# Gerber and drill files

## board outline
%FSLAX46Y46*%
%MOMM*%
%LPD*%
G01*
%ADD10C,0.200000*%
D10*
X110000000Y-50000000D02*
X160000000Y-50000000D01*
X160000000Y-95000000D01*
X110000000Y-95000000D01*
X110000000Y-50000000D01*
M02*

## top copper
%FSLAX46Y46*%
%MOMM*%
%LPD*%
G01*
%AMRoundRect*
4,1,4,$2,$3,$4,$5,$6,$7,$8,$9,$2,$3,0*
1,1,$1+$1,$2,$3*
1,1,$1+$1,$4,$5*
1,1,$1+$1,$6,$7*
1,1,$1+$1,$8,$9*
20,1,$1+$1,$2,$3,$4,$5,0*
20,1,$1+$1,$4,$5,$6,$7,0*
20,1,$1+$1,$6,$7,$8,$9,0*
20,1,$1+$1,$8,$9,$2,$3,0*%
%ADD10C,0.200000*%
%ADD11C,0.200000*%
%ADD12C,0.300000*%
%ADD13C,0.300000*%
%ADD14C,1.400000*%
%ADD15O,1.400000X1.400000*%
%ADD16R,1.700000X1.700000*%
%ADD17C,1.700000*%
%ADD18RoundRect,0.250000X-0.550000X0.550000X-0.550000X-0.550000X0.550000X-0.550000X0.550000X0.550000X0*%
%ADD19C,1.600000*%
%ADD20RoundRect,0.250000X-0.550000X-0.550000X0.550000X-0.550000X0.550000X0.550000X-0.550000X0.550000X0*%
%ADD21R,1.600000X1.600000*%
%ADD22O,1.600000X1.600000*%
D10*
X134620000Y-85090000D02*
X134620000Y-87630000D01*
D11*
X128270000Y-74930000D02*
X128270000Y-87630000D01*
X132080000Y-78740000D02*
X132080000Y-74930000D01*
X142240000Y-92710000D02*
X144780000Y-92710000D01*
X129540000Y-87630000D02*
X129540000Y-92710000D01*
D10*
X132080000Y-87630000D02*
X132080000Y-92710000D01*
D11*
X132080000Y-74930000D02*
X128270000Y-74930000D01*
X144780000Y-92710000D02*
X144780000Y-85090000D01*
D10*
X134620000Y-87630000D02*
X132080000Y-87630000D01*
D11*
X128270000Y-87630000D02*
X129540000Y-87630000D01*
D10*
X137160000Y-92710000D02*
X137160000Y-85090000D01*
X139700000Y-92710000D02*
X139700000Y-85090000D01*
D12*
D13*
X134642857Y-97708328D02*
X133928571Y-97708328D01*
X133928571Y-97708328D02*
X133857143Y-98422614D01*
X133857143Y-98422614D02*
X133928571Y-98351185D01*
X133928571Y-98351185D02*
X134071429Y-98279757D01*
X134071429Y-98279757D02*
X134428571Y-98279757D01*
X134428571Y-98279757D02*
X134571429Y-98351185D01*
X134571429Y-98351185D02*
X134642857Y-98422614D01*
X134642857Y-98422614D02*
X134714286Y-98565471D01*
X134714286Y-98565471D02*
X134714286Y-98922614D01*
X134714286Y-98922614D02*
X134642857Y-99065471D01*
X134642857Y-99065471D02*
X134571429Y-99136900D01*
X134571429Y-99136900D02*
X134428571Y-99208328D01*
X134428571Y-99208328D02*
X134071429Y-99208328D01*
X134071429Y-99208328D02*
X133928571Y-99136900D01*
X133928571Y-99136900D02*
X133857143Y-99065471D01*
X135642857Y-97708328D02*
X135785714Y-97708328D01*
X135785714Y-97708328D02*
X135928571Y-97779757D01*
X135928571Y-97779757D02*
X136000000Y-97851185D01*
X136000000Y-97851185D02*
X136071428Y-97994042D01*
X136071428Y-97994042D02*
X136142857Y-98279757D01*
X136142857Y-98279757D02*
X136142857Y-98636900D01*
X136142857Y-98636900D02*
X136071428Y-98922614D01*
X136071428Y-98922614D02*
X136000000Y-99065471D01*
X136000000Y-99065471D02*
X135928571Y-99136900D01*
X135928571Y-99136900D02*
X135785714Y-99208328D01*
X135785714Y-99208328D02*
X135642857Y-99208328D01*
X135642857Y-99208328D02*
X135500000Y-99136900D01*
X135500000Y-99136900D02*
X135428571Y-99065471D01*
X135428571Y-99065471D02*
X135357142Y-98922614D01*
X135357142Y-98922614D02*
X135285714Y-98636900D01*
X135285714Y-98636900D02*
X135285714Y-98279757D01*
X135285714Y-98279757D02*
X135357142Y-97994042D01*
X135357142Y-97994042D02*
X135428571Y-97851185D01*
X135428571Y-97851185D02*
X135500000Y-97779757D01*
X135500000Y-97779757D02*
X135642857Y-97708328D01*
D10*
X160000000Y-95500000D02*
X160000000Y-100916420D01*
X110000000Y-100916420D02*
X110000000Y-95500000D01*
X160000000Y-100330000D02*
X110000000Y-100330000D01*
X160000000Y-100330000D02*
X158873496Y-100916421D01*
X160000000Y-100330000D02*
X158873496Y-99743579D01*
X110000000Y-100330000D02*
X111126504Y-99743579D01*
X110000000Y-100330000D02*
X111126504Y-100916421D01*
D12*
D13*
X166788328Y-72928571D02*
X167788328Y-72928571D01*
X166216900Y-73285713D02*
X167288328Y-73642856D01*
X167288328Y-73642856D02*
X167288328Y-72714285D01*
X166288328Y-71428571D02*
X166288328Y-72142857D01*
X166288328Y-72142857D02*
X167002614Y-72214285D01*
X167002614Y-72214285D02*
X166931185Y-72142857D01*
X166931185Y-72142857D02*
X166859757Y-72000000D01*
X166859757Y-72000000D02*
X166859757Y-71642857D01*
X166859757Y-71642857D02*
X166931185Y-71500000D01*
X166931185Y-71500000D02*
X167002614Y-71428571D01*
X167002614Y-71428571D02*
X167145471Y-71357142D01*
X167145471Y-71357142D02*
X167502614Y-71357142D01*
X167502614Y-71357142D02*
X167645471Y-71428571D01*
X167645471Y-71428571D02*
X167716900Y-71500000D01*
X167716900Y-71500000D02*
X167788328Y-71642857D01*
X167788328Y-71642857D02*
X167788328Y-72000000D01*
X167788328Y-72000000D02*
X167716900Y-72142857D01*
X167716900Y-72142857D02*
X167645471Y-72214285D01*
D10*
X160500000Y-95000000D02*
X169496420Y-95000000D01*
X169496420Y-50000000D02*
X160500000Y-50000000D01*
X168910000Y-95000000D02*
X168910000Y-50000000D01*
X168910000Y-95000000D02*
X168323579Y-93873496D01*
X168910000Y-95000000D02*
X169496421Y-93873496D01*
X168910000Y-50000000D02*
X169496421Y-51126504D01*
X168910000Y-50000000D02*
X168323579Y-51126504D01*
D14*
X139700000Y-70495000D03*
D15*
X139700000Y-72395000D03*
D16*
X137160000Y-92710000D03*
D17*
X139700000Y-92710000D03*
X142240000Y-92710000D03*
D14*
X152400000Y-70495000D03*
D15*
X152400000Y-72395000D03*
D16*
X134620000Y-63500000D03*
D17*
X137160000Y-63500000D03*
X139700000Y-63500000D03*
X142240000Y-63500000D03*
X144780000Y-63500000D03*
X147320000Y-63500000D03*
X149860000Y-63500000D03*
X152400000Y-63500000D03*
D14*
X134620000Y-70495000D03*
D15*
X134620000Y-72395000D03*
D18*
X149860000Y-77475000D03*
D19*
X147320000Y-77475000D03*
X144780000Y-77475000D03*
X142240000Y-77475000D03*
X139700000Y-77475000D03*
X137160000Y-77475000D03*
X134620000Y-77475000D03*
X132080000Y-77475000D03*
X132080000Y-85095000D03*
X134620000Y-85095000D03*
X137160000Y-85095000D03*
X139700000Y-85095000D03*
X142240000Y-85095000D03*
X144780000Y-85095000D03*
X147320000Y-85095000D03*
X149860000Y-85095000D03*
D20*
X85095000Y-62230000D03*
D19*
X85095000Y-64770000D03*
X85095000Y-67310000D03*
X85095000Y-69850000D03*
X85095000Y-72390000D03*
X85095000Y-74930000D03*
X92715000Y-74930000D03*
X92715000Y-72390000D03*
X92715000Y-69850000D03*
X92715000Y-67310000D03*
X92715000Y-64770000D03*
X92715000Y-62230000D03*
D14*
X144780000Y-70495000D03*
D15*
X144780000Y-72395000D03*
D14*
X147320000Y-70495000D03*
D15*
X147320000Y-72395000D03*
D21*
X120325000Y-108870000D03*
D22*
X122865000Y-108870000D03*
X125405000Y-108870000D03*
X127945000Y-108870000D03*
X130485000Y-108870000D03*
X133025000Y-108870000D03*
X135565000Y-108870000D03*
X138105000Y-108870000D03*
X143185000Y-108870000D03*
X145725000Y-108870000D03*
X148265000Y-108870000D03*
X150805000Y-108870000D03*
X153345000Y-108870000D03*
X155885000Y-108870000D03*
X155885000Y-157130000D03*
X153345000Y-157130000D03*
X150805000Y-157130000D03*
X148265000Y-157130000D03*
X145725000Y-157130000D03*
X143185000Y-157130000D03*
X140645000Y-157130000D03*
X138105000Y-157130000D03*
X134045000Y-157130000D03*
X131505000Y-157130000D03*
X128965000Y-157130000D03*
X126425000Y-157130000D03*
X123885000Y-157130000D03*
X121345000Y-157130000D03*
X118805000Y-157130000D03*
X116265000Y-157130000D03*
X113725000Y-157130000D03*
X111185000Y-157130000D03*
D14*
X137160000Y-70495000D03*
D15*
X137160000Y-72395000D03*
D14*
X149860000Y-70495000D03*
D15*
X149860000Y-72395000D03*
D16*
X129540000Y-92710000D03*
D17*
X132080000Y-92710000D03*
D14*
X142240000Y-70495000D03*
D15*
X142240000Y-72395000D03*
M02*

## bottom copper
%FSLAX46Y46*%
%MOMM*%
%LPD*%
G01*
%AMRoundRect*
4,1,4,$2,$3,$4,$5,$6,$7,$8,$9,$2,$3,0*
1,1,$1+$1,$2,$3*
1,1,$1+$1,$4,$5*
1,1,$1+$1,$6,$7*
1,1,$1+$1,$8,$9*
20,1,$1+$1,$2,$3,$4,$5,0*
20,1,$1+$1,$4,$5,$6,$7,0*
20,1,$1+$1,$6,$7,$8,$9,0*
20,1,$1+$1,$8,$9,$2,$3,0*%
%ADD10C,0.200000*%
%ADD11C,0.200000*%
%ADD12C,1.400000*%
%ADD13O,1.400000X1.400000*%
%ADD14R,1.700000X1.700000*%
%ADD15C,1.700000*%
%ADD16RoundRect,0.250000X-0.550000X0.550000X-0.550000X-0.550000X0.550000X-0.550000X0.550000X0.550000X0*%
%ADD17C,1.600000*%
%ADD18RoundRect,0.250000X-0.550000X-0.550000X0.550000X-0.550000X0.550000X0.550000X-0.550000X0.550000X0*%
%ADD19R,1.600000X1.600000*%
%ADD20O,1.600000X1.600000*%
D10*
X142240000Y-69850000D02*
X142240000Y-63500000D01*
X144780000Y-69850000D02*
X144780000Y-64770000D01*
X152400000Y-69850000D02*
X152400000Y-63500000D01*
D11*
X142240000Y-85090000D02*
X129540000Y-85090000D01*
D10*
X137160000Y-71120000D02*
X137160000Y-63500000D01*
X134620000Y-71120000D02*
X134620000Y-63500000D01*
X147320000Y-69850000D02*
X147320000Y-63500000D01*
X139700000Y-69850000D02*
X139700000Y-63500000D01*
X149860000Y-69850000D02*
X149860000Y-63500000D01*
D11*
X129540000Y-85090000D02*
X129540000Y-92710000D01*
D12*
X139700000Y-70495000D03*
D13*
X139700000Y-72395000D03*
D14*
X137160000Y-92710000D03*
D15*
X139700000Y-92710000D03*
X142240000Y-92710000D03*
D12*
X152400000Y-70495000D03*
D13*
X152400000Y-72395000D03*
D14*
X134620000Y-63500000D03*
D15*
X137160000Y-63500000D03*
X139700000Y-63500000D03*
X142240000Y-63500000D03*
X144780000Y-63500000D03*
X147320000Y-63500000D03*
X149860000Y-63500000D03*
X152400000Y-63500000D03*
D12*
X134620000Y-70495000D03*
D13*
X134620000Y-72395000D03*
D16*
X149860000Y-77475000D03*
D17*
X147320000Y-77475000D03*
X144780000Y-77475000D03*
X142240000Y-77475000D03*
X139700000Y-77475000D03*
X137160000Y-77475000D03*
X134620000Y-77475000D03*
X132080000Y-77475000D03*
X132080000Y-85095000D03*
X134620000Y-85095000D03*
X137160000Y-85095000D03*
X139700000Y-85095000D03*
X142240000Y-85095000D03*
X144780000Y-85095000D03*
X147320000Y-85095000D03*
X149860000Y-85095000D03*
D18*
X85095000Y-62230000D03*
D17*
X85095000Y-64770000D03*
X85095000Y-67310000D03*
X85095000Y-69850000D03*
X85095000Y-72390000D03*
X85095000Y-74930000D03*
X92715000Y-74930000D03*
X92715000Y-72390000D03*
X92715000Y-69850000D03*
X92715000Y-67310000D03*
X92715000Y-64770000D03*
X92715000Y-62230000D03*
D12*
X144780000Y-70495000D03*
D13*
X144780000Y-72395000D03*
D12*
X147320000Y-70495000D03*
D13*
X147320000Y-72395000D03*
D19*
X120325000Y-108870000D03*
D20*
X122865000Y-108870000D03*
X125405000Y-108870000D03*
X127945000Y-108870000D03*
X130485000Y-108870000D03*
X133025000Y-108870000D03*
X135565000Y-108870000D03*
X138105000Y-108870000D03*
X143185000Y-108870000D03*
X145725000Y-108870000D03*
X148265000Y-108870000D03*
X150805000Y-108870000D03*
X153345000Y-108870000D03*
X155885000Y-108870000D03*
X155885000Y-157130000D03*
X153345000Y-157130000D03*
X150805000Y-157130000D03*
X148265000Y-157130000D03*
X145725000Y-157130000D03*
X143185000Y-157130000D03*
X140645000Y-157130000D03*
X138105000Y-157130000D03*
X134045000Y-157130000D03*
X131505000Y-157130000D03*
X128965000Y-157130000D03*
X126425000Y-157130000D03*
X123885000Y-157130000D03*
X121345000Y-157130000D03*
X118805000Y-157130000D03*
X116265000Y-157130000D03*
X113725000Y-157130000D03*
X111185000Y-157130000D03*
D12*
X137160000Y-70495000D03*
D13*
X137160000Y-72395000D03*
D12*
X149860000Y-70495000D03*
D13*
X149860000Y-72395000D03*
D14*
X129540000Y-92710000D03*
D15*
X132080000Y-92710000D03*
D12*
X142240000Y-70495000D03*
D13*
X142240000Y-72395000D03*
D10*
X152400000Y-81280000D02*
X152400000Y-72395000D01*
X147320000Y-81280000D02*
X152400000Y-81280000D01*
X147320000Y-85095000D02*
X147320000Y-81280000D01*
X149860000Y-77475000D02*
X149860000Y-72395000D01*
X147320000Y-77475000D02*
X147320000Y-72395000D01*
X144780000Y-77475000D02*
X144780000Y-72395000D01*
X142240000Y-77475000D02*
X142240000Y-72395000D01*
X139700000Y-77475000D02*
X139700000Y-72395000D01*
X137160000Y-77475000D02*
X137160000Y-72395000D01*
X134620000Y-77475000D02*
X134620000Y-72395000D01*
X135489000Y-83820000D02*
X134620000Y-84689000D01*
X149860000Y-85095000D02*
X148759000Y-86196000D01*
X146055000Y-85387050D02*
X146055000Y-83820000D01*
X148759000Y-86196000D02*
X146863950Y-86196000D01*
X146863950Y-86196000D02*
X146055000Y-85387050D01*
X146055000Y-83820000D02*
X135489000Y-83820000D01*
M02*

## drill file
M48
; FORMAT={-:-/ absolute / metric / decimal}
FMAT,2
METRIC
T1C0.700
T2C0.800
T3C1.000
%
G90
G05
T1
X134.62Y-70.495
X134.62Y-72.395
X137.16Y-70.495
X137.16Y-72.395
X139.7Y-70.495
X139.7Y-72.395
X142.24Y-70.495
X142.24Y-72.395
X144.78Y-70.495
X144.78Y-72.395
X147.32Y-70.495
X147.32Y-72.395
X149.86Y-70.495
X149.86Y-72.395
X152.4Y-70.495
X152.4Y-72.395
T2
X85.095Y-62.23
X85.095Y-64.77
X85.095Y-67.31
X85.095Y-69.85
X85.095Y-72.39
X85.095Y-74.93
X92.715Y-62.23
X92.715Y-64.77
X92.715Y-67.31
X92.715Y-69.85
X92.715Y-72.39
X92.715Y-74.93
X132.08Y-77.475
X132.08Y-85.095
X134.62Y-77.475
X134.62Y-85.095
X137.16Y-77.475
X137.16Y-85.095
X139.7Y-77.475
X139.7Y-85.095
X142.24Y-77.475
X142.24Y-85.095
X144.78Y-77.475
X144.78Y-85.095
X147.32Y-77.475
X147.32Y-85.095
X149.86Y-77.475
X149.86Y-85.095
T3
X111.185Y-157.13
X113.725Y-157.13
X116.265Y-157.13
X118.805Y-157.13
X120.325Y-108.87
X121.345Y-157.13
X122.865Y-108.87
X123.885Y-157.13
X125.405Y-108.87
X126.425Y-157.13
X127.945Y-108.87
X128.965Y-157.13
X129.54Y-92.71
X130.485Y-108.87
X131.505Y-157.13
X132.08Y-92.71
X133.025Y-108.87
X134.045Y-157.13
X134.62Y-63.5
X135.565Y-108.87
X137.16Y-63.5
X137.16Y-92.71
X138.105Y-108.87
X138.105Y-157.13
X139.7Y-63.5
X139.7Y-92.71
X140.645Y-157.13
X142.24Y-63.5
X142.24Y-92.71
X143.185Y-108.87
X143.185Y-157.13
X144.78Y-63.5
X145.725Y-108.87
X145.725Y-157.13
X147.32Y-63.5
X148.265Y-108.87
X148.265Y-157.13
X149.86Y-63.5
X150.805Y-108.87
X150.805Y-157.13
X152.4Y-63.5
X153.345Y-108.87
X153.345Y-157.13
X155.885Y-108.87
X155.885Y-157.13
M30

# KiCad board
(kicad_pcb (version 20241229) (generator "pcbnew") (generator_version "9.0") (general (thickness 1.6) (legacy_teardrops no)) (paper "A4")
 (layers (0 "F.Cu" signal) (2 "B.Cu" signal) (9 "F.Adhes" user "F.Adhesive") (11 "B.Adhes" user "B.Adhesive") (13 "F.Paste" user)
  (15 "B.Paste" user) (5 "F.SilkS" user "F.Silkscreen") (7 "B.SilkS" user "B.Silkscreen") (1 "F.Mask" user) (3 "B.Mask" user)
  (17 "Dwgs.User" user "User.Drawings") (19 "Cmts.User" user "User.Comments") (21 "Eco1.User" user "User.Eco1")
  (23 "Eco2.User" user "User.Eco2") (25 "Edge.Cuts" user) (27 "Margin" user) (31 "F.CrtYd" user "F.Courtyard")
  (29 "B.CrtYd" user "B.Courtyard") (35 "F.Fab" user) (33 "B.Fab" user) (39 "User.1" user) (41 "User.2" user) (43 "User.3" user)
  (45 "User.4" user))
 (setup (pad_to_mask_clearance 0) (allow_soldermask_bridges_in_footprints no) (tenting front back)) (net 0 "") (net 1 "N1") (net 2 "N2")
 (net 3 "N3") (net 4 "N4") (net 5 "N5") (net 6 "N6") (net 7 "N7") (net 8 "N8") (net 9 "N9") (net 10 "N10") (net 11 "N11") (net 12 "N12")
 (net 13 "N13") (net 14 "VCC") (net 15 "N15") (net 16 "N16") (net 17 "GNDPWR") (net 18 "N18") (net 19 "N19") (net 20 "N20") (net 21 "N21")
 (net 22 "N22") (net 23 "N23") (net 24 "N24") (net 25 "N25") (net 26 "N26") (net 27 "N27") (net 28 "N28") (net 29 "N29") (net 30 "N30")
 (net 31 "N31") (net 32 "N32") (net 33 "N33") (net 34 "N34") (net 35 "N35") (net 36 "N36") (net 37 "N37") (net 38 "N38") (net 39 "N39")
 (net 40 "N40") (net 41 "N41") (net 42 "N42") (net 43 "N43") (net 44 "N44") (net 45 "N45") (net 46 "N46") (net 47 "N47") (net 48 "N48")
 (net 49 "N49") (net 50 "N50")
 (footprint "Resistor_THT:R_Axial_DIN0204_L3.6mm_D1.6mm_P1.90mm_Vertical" (layer "F.Cu") (at 139.7 70.495 -90)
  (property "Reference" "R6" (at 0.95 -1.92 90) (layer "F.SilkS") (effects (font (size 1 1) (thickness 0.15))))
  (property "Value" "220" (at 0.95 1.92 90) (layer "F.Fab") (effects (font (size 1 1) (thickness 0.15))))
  (pad "1" thru_hole circle (at 0 0 270) (size 1.4 1.4) (drill 0.7) (layers "*.Cu" "*.Mask") (remove_unused_layers no) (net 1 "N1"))
  (pad "2" thru_hole oval (at 1.9 0 270) (size 1.4 1.4) (drill 0.7) (layers "*.Cu" "*.Mask") (remove_unused_layers no) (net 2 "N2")))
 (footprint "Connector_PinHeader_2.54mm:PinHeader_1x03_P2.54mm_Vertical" (layer "F.Cu") (at 137.16 92.71 90)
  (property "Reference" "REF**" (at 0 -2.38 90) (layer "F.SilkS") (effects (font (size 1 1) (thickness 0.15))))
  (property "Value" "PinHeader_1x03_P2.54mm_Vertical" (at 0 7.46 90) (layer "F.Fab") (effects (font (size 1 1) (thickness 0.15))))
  (pad "1" thru_hole rect (at 0 0 90) (size 1.7 1.7) (drill 1) (layers "*.Cu" "*.Mask") (remove_unused_layers no))
  (pad "2" thru_hole circle (at 0 2.54 90) (size 1.7 1.7) (drill 1) (layers "*.Cu" "*.Mask") (remove_unused_layers no))
  (pad "3" thru_hole circle (at 0 5.08 90) (size 1.7 1.7) (drill 1) (layers "*.Cu" "*.Mask") (remove_unused_layers no)))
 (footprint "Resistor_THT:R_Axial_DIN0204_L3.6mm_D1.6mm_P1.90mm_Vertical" (layer "F.Cu") (at 152.4 70.495 -90)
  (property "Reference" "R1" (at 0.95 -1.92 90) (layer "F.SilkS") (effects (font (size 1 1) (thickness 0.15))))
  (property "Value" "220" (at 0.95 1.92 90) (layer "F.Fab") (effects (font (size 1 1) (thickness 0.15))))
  (pad "1" thru_hole circle (at 0 0 270) (size 1.4 1.4) (drill 0.7) (layers "*.Cu" "*.Mask") (remove_unused_layers no) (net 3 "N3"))
  (pad "2" thru_hole oval (at 1.9 0 270) (size 1.4 1.4) (drill 0.7) (layers "*.Cu" "*.Mask") (remove_unused_layers no) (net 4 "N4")))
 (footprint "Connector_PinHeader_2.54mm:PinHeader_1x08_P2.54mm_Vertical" (layer "F.Cu") (at 134.62 63.5 90)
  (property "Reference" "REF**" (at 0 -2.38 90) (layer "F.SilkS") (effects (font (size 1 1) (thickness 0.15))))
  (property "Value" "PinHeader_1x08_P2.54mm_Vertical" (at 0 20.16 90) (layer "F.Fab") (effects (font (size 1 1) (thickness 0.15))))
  (pad "1" thru_hole rect (at 0 0 90) (size 1.7 1.7) (drill 1) (layers "*.Cu" "*.Mask") (remove_unused_layers no))
  (pad "2" thru_hole circle (at 0 2.54 90) (size 1.7 1.7) (drill 1) (layers "*.Cu" "*.Mask") (remove_unused_layers no))
  (pad "3" thru_hole circle (at 0 5.08 90) (size 1.7 1.7) (drill 1) (layers "*.Cu" "*.Mask") (remove_unused_layers no))
  (pad "4" thru_hole circle (at 0 7.62 90) (size 1.7 1.7) (drill 1) (layers "*.Cu" "*.Mask") (remove_unused_layers no))
  (pad "5" thru_hole circle (at 0 10.16 90) (size 1.7 1.7) (drill 1) (layers "*.Cu" "*.Mask") (remove_unused_layers no))
  (pad "6" thru_hole circle (at 0 12.7 90) (size 1.7 1.7) (drill 1) (layers "*.Cu" "*.Mask") (remove_unused_layers no))
  (pad "7" thru_hole circle (at 0 15.24 90) (size 1.7 1.7) (drill 1) (layers "*.Cu" "*.Mask") (remove_unused_layers no))
  (pad "8" thru_hole circle (at 0 17.78 90) (size 1.7 1.7) (drill 1) (layers "*.Cu" "*.Mask") (remove_unused_layers no)))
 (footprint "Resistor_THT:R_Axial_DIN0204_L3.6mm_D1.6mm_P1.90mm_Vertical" (layer "F.Cu") (at 134.62 70.495 -90)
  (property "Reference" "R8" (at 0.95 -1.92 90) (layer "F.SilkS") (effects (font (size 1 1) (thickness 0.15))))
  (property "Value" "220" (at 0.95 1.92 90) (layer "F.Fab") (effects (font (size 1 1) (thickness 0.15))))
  (pad "1" thru_hole circle (at 0 0 270) (size 1.4 1.4) (drill 0.7) (layers "*.Cu" "*.Mask") (remove_unused_layers no) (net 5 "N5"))
  (pad "2" thru_hole oval (at 1.9 0 270) (size 1.4 1.4) (drill 0.7) (layers "*.Cu" "*.Mask") (remove_unused_layers no) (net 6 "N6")))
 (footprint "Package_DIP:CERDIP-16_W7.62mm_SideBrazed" (layer "F.Cu") (at 149.86 77.475 -90)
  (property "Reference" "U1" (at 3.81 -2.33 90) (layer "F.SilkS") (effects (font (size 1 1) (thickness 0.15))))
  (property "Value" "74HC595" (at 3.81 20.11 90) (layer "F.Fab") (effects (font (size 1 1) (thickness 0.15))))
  (pad "1" thru_hole roundrect (at 0 0 270) (size 1.6 1.6) (drill 0.8) (layers "*.Cu" "*.Mask") (remove_unused_layers no)
   (roundrect_rratio 0.15625) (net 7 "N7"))
  (pad "2" thru_hole circle (at 0 2.54 270) (size 1.6 1.6) (drill 0.8) (layers "*.Cu" "*.Mask") (remove_unused_layers no) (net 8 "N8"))
  (pad "3" thru_hole circle (at 0 5.08 270) (size 1.6 1.6) (drill 0.8) (layers "*.Cu" "*.Mask") (remove_unused_layers no) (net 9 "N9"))
  (pad "4" thru_hole circle (at 0 7.62 270) (size 1.6 1.6) (drill 0.8) (layers "*.Cu" "*.Mask") (remove_unused_layers no) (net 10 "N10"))
  (pad "5" thru_hole circle (at 0 10.16 270) (size 1.6 1.6) (drill 0.8) (layers "*.Cu" "*.Mask") (remove_unused_layers no) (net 2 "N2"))
  (pad "6" thru_hole circle (at 0 12.7 270) (size 1.6 1.6) (drill 0.8) (layers "*.Cu" "*.Mask") (remove_unused_layers no) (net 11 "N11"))
  (pad "7" thru_hole circle (at 0 15.24 270) (size 1.6 1.6) (drill 0.8) (layers "*.Cu" "*.Mask") (remove_unused_layers no) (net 6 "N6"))
  (pad "8" thru_hole circle (at 0 17.78 270) (size 1.6 1.6) (drill 0.8) (layers "*.Cu" "*.Mask") (remove_unused_layers no) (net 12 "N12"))
  (pad "9" thru_hole circle (at 7.62 17.78 270) (size 1.6 1.6) (drill 0.8) (layers "*.Cu" "*.Mask") (remove_unused_layers no) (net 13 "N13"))
  (pad "10" thru_hole circle (at 7.62 15.24 270) (size 1.6 1.6) (drill 0.8) (layers "*.Cu" "*.Mask") (remove_unused_layers no)
   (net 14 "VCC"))
  (pad "11" thru_hole circle (at 7.62 12.7 270) (size 1.6 1.6) (drill 0.8) (layers "*.Cu" "*.Mask") (remove_unused_layers no) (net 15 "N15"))
  (pad "12" thru_hole circle (at 7.62 10.16 270) (size 1.6 1.6) (drill 0.8) (layers "*.Cu" "*.Mask") (remove_unused_layers no)
   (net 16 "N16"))
  (pad "13" thru_hole circle (at 7.62 7.62 270) (size 1.6 1.6) (drill 0.8) (layers "*.Cu" "*.Mask") (remove_unused_layers no)
   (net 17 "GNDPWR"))
  (pad "14" thru_hole circle (at 7.62 5.08 270) (size 1.6 1.6) (drill 0.8) (layers "*.Cu" "*.Mask") (remove_unused_layers no) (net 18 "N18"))
  (pad "15" thru_hole circle (at 7.62 2.54 270) (size 1.6 1.6) (drill 0.8) (layers "*.Cu" "*.Mask") (remove_unused_layers no) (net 4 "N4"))
  (pad "16" thru_hole circle (at 7.62 0 270) (size 1.6 1.6) (drill 0.8) (layers "*.Cu" "*.Mask") (remove_unused_layers no) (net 14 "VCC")))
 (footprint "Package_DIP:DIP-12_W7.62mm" (layer "F.Cu") (at 85.095 62.23)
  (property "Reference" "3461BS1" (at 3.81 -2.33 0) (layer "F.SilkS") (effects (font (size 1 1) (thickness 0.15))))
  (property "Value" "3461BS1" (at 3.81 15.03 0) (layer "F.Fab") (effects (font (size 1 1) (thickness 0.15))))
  (pad "1" thru_hole roundrect (at 0 0) (size 1.6 1.6) (drill 0.8) (layers "*.Cu" "*.Mask") (remove_unused_layers no)
   (roundrect_rratio 0.15625) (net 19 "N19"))
  (pad "2" thru_hole circle (at 0 2.54) (size 1.6 1.6) (drill 0.8) (layers "*.Cu" "*.Mask") (remove_unused_layers no) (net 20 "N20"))
  (pad "3" thru_hole circle (at 0 5.08) (size 1.6 1.6) (drill 0.8) (layers "*.Cu" "*.Mask") (remove_unused_layers no) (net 5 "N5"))
  (pad "4" thru_hole circle (at 0 7.62) (size 1.6 1.6) (drill 0.8) (layers "*.Cu" "*.Mask") (remove_unused_layers no) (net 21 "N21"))
  (pad "5" thru_hole circle (at 0 10.16) (size 1.6 1.6) (drill 0.8) (layers "*.Cu" "*.Mask") (remove_unused_layers no) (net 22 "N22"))
  (pad "6" thru_hole circle (at 0 12.7) (size 1.6 1.6) (drill 0.8) (layers "*.Cu" "*.Mask") (remove_unused_layers no) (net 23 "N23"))
  (pad "7" thru_hole circle (at 7.62 12.7) (size 1.6 1.6) (drill 0.8) (layers "*.Cu" "*.Mask") (remove_unused_layers no) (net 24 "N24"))
  (pad "8" thru_hole circle (at 7.62 10.16) (size 1.6 1.6) (drill 0.8) (layers "*.Cu" "*.Mask") (remove_unused_layers no) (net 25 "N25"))
  (pad "9" thru_hole circle (at 7.62 7.62) (size 1.6 1.6) (drill 0.8) (layers "*.Cu" "*.Mask") (remove_unused_layers no) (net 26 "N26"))
  (pad "10" thru_hole circle (at 7.62 5.08) (size 1.6 1.6) (drill 0.8) (layers "*.Cu" "*.Mask") (remove_unused_layers no) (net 1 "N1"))
  (pad "11" thru_hole circle (at 7.62 2.54) (size 1.6 1.6) (drill 0.8) (layers "*.Cu" "*.Mask") (remove_unused_layers no) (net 3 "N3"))
  (pad "12" thru_hole circle (at 7.62 0) (size 1.6 1.6) (drill 0.8) (layers "*.Cu" "*.Mask") (remove_unused_layers no) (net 17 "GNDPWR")))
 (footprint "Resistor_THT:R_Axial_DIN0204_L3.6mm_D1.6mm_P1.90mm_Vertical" (layer "F.Cu") (at 144.78 70.495 -90)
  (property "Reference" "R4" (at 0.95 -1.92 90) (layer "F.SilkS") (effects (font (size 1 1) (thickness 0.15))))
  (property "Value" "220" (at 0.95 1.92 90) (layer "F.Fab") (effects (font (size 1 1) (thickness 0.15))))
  (pad "1" thru_hole circle (at 0 0 270) (size 1.4 1.4) (drill 0.7) (layers "*.Cu" "*.Mask") (remove_unused_layers no) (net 20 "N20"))
  (pad "2" thru_hole oval (at 1.9 0 270) (size 1.4 1.4) (drill 0.7) (layers "*.Cu" "*.Mask") (remove_unused_layers no) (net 9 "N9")))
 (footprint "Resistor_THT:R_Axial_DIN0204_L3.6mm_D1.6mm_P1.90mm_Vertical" (layer "F.Cu") (at 147.32 70.495 -90)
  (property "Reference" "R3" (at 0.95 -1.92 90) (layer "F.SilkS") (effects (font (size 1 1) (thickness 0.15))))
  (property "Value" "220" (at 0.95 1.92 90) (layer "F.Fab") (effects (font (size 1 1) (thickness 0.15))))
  (pad "1" thru_hole circle (at 0 0 270) (size 1.4 1.4) (drill 0.7) (layers "*.Cu" "*.Mask") (remove_unused_layers no) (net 21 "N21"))
  (pad "2" thru_hole oval (at 1.9 0 270) (size 1.4 1.4) (drill 0.7) (layers "*.Cu" "*.Mask") (remove_unused_layers no) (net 8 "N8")))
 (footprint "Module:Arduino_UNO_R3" (layer "F.Cu") (at 120.325 108.87)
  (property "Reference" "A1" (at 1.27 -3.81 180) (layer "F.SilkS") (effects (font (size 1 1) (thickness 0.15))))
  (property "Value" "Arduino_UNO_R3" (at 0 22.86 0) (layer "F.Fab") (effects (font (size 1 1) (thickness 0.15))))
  (pad "1" thru_hole rect (at 0 0 90) (size 1.6 1.6) (drill 1) (layers "*.Cu" "*.Mask") (remove_unused_layers no) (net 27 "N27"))
  (pad "2" thru_hole oval (at 2.54 0 90) (size 1.6 1.6) (drill 1) (layers "*.Cu" "*.Mask") (remove_unused_layers no) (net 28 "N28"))
  (pad "3" thru_hole oval (at 5.08 0 90) (size 1.6 1.6) (drill 1) (layers "*.Cu" "*.Mask") (remove_unused_layers no) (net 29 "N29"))
  (pad "4" thru_hole oval (at 7.62 0 90) (size 1.6 1.6) (drill 1) (layers "*.Cu" "*.Mask") (remove_unused_layers no) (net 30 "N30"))
  (pad "5" thru_hole oval (at 10.16 0 90) (size 1.6 1.6) (drill 1) (layers "*.Cu" "*.Mask") (remove_unused_layers no) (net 14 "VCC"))
  (pad "6" thru_hole oval (at 12.7 0 90) (size 1.6 1.6) (drill 1) (layers "*.Cu" "*.Mask") (remove_unused_layers no) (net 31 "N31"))
  (pad "7" thru_hole oval (at 15.24 0 90) (size 1.6 1.6) (drill 1) (layers "*.Cu" "*.Mask") (remove_unused_layers no) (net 17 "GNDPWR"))
  (pad "8" thru_hole oval (at 17.78 0 90) (size 1.6 1.6) (drill 1) (layers "*.Cu" "*.Mask") (remove_unused_layers no) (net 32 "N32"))
  (pad "9" thru_hole oval (at 22.86 0 90) (size 1.6 1.6) (drill 1) (layers "*.Cu" "*.Mask") (remove_unused_layers no) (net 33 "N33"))
  (pad "10" thru_hole oval (at 25.4 0 90) (size 1.6 1.6) (drill 1) (layers "*.Cu" "*.Mask") (remove_unused_layers no) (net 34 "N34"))
  (pad "11" thru_hole oval (at 27.94 0 90) (size 1.6 1.6) (drill 1) (layers "*.Cu" "*.Mask") (remove_unused_layers no) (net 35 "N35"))
  (pad "12" thru_hole oval (at 30.48 0 90) (size 1.6 1.6) (drill 1) (layers "*.Cu" "*.Mask") (remove_unused_layers no) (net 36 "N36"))
  (pad "13" thru_hole oval (at 33.02 0 90) (size 1.6 1.6) (drill 1) (layers "*.Cu" "*.Mask") (remove_unused_layers no) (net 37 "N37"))
  (pad "14" thru_hole oval (at 35.56 0 90) (size 1.6 1.6) (drill 1) (layers "*.Cu" "*.Mask") (remove_unused_layers no) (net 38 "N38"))
  (pad "15" thru_hole oval (at 35.56 48.26 90) (size 1.6 1.6) (drill 1) (layers "*.Cu" "*.Mask") (remove_unused_layers no) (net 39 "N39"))
  (pad "16" thru_hole oval (at 33.02 48.26 90) (size 1.6 1.6) (drill 1) (layers "*.Cu" "*.Mask") (remove_unused_layers no) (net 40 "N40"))
  (pad "17" thru_hole oval (at 30.48 48.26 90) (size 1.6 1.6) (drill 1) (layers "*.Cu" "*.Mask") (remove_unused_layers no) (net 23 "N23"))
  (pad "18" thru_hole oval (at 27.94 48.26 90) (size 1.6 1.6) (drill 1) (layers "*.Cu" "*.Mask") (remove_unused_layers no) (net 25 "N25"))
  (pad "19" thru_hole oval (at 25.4 48.26 90) (size 1.6 1.6) (drill 1) (layers "*.Cu" "*.Mask") (remove_unused_layers no) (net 26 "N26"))
  (pad "20" thru_hole oval (at 22.86 48.26 90) (size 1.6 1.6) (drill 1) (layers "*.Cu" "*.Mask") (remove_unused_layers no) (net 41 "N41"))
  (pad "21" thru_hole oval (at 20.32 48.26 90) (size 1.6 1.6) (drill 1) (layers "*.Cu" "*.Mask") (remove_unused_layers no) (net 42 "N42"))
  (pad "22" thru_hole oval (at 17.78 48.26 90) (size 1.6 1.6) (drill 1) (layers "*.Cu" "*.Mask") (remove_unused_layers no) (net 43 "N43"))
  (pad "23" thru_hole oval (at 13.72 48.26 90) (size 1.6 1.6) (drill 1) (layers "*.Cu" "*.Mask") (remove_unused_layers no) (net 16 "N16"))
  (pad "24" thru_hole oval (at 11.18 48.26 90) (size 1.6 1.6) (drill 1) (layers "*.Cu" "*.Mask") (remove_unused_layers no) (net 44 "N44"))
  (pad "25" thru_hole oval (at 8.64 48.26 90) (size 1.6 1.6) (drill 1) (layers "*.Cu" "*.Mask") (remove_unused_layers no) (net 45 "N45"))
  (pad "26" thru_hole oval (at 6.1 48.26 90) (size 1.6 1.6) (drill 1) (layers "*.Cu" "*.Mask") (remove_unused_layers no) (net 18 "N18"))
  (pad "27" thru_hole oval (at 3.56 48.26 90) (size 1.6 1.6) (drill 1) (layers "*.Cu" "*.Mask") (remove_unused_layers no) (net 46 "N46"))
  (pad "28" thru_hole oval (at 1.02 48.26 90) (size 1.6 1.6) (drill 1) (layers "*.Cu" "*.Mask") (remove_unused_layers no) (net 15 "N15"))
  (pad "29" thru_hole oval (at -1.52 48.26 90) (size 1.6 1.6) (drill 1) (layers "*.Cu" "*.Mask") (remove_unused_layers no) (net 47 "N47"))
  (pad "30" thru_hole oval (at -4.06 48.26 90) (size 1.6 1.6) (drill 1) (layers "*.Cu" "*.Mask") (remove_unused_layers no) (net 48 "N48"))
  (pad "31" thru_hole oval (at -6.6 48.26 90) (size 1.6 1.6) (drill 1) (layers "*.Cu" "*.Mask") (remove_unused_layers no) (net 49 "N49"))
  (pad "32" thru_hole oval (at -9.14 48.26 90) (size 1.6 1.6) (drill 1) (layers "*.Cu" "*.Mask") (remove_unused_layers no) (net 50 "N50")))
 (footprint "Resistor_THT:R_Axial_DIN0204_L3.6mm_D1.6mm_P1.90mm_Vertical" (layer "F.Cu") (at 137.16 70.495 -90)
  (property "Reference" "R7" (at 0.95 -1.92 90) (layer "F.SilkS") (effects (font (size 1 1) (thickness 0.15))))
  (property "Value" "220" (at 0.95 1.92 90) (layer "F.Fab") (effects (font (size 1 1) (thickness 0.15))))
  (pad "1" thru_hole circle (at 0 0 270) (size 1.4 1.4) (drill 0.7) (layers "*.Cu" "*.Mask") (remove_unused_layers no) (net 22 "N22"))
  (pad "2" thru_hole oval (at 1.9 0 270) (size 1.4 1.4) (drill 0.7) (layers "*.Cu" "*.Mask") (remove_unused_layers no) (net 11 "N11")))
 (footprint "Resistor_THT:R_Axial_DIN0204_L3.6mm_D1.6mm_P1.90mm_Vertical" (layer "F.Cu") (at 149.86 70.495 -90)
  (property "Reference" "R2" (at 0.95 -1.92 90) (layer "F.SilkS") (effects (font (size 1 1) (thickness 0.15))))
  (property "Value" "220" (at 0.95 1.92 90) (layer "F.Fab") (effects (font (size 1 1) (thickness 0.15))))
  (pad "1" thru_hole circle (at 0 0 270) (size 1.4 1.4) (drill 0.7) (layers "*.Cu" "*.Mask") (remove_unused_layers no) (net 24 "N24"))
  (pad "2" thru_hole oval (at 1.9 0 270) (size 1.4 1.4) (drill 0.7) (layers "*.Cu" "*.Mask") (remove_unused_layers no) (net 7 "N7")))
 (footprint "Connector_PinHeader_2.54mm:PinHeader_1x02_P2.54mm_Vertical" (layer "F.Cu") (at 129.54 92.71 90)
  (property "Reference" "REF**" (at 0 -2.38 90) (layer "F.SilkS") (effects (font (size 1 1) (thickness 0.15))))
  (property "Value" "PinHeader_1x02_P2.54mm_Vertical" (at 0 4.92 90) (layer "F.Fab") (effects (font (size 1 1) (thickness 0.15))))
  (pad "1" thru_hole rect (at 0 0 90) (size 1.7 1.7) (drill 1) (layers "*.Cu" "*.Mask") (remove_unused_layers no))
  (pad "2" thru_hole circle (at 0 2.54 90) (size 1.7 1.7) (drill 1) (layers "*.Cu" "*.Mask") (remove_unused_layers no)))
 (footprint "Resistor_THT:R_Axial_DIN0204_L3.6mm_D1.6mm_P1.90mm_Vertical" (layer "F.Cu") (at 142.24 70.495 -90)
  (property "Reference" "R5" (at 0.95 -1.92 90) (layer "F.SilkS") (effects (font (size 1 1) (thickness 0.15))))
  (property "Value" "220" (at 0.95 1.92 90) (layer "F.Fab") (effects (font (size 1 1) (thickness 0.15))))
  (pad "1" thru_hole circle (at 0 0 270) (size 1.4 1.4) (drill 0.7) (layers "*.Cu" "*.Mask") (remove_unused_layers no) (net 19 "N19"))
  (pad "2" thru_hole oval (at 1.9 0 270) (size 1.4 1.4) (drill 0.7) (layers "*.Cu" "*.Mask") (remove_unused_layers no) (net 10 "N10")))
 (gr_line (start 134.62 85.09) (end 134.62 87.63) (stroke (width 0.2) (type default)) (layer "F.Cu"))
 (gr_line (start 128.27 74.93) (end 128.27 87.63) (stroke (width 0.2) (type default)) (layer "F.Cu") (net 12))
 (gr_line (start 132.08 78.74) (end 132.08 74.93) (stroke (width 0.2) (type default)) (layer "F.Cu") (net 12))
 (gr_line (start 142.24 92.71) (end 144.78 92.71) (stroke (width 0.2) (type default)) (layer "F.Cu") (net 18))
 (gr_line (start 129.54 87.63) (end 129.54 92.71) (stroke (width 0.2) (type default)) (layer "F.Cu") (net 12))
 (gr_line (start 132.08 87.63) (end 132.08 92.71) (stroke (width 0.2) (type default)) (layer "F.Cu"))
 (gr_line (start 132.08 74.93) (end 128.27 74.93) (stroke (width 0.2) (type default)) (layer "F.Cu") (net 12))
 (gr_line (start 144.78 92.71) (end 144.78 85.09) (stroke (width 0.2) (type default)) (layer "F.Cu") (net 18))
 (gr_line (start 134.62 87.63) (end 132.08 87.63) (stroke (width 0.2) (type default)) (layer "F.Cu"))
 (gr_line (start 128.27 87.63) (end 129.54 87.63) (stroke (width 0.2) (type default)) (layer "F.Cu") (net 12))
 (gr_line (start 137.16 92.71) (end 137.16 85.09) (stroke (width 0.2) (type default)) (layer "F.Cu"))
 (gr_line (start 139.7 92.71) (end 139.7 85.09) (stroke (width 0.2) (type default)) (layer "F.Cu"))
 (gr_line (start 142.24 69.85) (end 142.24 63.5) (stroke (width 0.2) (type default)) (layer "B.Cu") (net 19))
 (gr_line (start 144.78 69.85) (end 144.78 64.77) (stroke (width 0.2) (type default)) (layer "B.Cu") (net 20))
 (gr_line (start 152.4 69.85) (end 152.4 63.5) (stroke (width 0.2) (type default)) (layer "B.Cu") (net 3))
 (gr_line (start 142.24 85.09) (end 129.54 85.09) (stroke (width 0.2) (type default)) (layer "B.Cu"))
 (gr_line (start 137.16 71.12) (end 137.16 63.5) (stroke (width 0.2) (type default)) (layer "B.Cu") (net 22))
 (gr_line (start 134.62 71.12) (end 134.62 63.5) (stroke (width 0.2) (type default)) (layer "B.Cu") (net 5))
 (gr_line (start 147.32 69.85) (end 147.32 63.5) (stroke (width 0.2) (type default)) (layer "B.Cu") (net 21))
 (gr_line (start 139.7 69.85) (end 139.7 63.5) (stroke (width 0.2) (type default)) (layer "B.Cu") (net 1))
 (gr_line (start 149.86 69.85) (end 149.86 63.5) (stroke (width 0.2) (type default)) (layer "B.Cu") (net 24))
 (gr_line (start 129.54 85.09) (end 129.54 92.71) (stroke (width 0.2) (type default)) (layer "B.Cu"))
 (gr_rect (start 110 50) (end 160 95) (stroke (width 0.2) (type solid)) (fill no) (layer "Edge.Cuts"))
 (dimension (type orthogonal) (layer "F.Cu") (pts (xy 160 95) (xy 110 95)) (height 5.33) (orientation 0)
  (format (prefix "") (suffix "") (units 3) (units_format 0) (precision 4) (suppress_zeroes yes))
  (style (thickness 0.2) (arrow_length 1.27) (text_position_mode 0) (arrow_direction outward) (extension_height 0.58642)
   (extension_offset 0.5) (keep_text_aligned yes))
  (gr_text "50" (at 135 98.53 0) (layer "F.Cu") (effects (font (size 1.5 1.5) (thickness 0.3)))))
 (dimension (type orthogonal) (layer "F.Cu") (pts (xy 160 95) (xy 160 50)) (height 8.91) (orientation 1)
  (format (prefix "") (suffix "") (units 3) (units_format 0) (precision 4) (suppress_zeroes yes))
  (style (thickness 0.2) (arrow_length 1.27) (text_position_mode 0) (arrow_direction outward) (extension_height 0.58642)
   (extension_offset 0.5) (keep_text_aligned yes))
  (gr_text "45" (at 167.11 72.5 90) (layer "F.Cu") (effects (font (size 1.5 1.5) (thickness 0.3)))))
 (segment (start 152.4 81.28) (end 152.4 72.395) (width 0.2) (layer "B.Cu") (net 4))
 (segment (start 147.32 81.28) (end 152.4 81.28) (width 0.2) (layer "B.Cu") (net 4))
 (segment (start 147.32 85.095) (end 147.32 81.28) (width 0.2) (layer "B.Cu") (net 4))
 (segment (start 149.86 77.475) (end 149.86 72.395) (width 0.2) (layer "B.Cu") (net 7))
 (segment (start 147.32 77.475) (end 147.32 72.395) (width 0.2) (layer "B.Cu") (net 8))
 (segment (start 144.78 77.475) (end 144.78 72.395) (width 0.2) (layer "B.Cu") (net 9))
 (segment (start 142.24 77.475) (end 142.24 72.395) (width 0.2) (layer "B.Cu") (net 10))
 (segment (start 139.7 77.475) (end 139.7 72.395) (width 0.2) (layer "B.Cu") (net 2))
 (segment (start 137.16 77.475) (end 137.16 72.395) (width 0.2) (layer "B.Cu") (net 11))
 (segment (start 134.62 77.475) (end 134.62 72.395) (width 0.2) (layer "B.Cu") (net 6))
 (segment (start 135.489 83.82) (end 134.62 84.689) (width 0.2) (layer "B.Cu") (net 14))
 (segment (start 149.86 85.095) (end 148.759 86.196) (width 0.2) (layer "B.Cu") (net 14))
 (segment (start 146.055 85.38705) (end 146.055 83.82) (width 0.2) (layer "B.Cu") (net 14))
 (segment (start 148.759 86.196) (end 146.86395 86.196) (width 0.2) (layer "B.Cu") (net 14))
 (segment (start 146.86395 86.196) (end 146.055 85.38705) (width 0.2) (layer "B.Cu") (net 14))
 (segment (start 146.055 83.82) (end 135.489 83.82) (width 0.2) (layer "B.Cu") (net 14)))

